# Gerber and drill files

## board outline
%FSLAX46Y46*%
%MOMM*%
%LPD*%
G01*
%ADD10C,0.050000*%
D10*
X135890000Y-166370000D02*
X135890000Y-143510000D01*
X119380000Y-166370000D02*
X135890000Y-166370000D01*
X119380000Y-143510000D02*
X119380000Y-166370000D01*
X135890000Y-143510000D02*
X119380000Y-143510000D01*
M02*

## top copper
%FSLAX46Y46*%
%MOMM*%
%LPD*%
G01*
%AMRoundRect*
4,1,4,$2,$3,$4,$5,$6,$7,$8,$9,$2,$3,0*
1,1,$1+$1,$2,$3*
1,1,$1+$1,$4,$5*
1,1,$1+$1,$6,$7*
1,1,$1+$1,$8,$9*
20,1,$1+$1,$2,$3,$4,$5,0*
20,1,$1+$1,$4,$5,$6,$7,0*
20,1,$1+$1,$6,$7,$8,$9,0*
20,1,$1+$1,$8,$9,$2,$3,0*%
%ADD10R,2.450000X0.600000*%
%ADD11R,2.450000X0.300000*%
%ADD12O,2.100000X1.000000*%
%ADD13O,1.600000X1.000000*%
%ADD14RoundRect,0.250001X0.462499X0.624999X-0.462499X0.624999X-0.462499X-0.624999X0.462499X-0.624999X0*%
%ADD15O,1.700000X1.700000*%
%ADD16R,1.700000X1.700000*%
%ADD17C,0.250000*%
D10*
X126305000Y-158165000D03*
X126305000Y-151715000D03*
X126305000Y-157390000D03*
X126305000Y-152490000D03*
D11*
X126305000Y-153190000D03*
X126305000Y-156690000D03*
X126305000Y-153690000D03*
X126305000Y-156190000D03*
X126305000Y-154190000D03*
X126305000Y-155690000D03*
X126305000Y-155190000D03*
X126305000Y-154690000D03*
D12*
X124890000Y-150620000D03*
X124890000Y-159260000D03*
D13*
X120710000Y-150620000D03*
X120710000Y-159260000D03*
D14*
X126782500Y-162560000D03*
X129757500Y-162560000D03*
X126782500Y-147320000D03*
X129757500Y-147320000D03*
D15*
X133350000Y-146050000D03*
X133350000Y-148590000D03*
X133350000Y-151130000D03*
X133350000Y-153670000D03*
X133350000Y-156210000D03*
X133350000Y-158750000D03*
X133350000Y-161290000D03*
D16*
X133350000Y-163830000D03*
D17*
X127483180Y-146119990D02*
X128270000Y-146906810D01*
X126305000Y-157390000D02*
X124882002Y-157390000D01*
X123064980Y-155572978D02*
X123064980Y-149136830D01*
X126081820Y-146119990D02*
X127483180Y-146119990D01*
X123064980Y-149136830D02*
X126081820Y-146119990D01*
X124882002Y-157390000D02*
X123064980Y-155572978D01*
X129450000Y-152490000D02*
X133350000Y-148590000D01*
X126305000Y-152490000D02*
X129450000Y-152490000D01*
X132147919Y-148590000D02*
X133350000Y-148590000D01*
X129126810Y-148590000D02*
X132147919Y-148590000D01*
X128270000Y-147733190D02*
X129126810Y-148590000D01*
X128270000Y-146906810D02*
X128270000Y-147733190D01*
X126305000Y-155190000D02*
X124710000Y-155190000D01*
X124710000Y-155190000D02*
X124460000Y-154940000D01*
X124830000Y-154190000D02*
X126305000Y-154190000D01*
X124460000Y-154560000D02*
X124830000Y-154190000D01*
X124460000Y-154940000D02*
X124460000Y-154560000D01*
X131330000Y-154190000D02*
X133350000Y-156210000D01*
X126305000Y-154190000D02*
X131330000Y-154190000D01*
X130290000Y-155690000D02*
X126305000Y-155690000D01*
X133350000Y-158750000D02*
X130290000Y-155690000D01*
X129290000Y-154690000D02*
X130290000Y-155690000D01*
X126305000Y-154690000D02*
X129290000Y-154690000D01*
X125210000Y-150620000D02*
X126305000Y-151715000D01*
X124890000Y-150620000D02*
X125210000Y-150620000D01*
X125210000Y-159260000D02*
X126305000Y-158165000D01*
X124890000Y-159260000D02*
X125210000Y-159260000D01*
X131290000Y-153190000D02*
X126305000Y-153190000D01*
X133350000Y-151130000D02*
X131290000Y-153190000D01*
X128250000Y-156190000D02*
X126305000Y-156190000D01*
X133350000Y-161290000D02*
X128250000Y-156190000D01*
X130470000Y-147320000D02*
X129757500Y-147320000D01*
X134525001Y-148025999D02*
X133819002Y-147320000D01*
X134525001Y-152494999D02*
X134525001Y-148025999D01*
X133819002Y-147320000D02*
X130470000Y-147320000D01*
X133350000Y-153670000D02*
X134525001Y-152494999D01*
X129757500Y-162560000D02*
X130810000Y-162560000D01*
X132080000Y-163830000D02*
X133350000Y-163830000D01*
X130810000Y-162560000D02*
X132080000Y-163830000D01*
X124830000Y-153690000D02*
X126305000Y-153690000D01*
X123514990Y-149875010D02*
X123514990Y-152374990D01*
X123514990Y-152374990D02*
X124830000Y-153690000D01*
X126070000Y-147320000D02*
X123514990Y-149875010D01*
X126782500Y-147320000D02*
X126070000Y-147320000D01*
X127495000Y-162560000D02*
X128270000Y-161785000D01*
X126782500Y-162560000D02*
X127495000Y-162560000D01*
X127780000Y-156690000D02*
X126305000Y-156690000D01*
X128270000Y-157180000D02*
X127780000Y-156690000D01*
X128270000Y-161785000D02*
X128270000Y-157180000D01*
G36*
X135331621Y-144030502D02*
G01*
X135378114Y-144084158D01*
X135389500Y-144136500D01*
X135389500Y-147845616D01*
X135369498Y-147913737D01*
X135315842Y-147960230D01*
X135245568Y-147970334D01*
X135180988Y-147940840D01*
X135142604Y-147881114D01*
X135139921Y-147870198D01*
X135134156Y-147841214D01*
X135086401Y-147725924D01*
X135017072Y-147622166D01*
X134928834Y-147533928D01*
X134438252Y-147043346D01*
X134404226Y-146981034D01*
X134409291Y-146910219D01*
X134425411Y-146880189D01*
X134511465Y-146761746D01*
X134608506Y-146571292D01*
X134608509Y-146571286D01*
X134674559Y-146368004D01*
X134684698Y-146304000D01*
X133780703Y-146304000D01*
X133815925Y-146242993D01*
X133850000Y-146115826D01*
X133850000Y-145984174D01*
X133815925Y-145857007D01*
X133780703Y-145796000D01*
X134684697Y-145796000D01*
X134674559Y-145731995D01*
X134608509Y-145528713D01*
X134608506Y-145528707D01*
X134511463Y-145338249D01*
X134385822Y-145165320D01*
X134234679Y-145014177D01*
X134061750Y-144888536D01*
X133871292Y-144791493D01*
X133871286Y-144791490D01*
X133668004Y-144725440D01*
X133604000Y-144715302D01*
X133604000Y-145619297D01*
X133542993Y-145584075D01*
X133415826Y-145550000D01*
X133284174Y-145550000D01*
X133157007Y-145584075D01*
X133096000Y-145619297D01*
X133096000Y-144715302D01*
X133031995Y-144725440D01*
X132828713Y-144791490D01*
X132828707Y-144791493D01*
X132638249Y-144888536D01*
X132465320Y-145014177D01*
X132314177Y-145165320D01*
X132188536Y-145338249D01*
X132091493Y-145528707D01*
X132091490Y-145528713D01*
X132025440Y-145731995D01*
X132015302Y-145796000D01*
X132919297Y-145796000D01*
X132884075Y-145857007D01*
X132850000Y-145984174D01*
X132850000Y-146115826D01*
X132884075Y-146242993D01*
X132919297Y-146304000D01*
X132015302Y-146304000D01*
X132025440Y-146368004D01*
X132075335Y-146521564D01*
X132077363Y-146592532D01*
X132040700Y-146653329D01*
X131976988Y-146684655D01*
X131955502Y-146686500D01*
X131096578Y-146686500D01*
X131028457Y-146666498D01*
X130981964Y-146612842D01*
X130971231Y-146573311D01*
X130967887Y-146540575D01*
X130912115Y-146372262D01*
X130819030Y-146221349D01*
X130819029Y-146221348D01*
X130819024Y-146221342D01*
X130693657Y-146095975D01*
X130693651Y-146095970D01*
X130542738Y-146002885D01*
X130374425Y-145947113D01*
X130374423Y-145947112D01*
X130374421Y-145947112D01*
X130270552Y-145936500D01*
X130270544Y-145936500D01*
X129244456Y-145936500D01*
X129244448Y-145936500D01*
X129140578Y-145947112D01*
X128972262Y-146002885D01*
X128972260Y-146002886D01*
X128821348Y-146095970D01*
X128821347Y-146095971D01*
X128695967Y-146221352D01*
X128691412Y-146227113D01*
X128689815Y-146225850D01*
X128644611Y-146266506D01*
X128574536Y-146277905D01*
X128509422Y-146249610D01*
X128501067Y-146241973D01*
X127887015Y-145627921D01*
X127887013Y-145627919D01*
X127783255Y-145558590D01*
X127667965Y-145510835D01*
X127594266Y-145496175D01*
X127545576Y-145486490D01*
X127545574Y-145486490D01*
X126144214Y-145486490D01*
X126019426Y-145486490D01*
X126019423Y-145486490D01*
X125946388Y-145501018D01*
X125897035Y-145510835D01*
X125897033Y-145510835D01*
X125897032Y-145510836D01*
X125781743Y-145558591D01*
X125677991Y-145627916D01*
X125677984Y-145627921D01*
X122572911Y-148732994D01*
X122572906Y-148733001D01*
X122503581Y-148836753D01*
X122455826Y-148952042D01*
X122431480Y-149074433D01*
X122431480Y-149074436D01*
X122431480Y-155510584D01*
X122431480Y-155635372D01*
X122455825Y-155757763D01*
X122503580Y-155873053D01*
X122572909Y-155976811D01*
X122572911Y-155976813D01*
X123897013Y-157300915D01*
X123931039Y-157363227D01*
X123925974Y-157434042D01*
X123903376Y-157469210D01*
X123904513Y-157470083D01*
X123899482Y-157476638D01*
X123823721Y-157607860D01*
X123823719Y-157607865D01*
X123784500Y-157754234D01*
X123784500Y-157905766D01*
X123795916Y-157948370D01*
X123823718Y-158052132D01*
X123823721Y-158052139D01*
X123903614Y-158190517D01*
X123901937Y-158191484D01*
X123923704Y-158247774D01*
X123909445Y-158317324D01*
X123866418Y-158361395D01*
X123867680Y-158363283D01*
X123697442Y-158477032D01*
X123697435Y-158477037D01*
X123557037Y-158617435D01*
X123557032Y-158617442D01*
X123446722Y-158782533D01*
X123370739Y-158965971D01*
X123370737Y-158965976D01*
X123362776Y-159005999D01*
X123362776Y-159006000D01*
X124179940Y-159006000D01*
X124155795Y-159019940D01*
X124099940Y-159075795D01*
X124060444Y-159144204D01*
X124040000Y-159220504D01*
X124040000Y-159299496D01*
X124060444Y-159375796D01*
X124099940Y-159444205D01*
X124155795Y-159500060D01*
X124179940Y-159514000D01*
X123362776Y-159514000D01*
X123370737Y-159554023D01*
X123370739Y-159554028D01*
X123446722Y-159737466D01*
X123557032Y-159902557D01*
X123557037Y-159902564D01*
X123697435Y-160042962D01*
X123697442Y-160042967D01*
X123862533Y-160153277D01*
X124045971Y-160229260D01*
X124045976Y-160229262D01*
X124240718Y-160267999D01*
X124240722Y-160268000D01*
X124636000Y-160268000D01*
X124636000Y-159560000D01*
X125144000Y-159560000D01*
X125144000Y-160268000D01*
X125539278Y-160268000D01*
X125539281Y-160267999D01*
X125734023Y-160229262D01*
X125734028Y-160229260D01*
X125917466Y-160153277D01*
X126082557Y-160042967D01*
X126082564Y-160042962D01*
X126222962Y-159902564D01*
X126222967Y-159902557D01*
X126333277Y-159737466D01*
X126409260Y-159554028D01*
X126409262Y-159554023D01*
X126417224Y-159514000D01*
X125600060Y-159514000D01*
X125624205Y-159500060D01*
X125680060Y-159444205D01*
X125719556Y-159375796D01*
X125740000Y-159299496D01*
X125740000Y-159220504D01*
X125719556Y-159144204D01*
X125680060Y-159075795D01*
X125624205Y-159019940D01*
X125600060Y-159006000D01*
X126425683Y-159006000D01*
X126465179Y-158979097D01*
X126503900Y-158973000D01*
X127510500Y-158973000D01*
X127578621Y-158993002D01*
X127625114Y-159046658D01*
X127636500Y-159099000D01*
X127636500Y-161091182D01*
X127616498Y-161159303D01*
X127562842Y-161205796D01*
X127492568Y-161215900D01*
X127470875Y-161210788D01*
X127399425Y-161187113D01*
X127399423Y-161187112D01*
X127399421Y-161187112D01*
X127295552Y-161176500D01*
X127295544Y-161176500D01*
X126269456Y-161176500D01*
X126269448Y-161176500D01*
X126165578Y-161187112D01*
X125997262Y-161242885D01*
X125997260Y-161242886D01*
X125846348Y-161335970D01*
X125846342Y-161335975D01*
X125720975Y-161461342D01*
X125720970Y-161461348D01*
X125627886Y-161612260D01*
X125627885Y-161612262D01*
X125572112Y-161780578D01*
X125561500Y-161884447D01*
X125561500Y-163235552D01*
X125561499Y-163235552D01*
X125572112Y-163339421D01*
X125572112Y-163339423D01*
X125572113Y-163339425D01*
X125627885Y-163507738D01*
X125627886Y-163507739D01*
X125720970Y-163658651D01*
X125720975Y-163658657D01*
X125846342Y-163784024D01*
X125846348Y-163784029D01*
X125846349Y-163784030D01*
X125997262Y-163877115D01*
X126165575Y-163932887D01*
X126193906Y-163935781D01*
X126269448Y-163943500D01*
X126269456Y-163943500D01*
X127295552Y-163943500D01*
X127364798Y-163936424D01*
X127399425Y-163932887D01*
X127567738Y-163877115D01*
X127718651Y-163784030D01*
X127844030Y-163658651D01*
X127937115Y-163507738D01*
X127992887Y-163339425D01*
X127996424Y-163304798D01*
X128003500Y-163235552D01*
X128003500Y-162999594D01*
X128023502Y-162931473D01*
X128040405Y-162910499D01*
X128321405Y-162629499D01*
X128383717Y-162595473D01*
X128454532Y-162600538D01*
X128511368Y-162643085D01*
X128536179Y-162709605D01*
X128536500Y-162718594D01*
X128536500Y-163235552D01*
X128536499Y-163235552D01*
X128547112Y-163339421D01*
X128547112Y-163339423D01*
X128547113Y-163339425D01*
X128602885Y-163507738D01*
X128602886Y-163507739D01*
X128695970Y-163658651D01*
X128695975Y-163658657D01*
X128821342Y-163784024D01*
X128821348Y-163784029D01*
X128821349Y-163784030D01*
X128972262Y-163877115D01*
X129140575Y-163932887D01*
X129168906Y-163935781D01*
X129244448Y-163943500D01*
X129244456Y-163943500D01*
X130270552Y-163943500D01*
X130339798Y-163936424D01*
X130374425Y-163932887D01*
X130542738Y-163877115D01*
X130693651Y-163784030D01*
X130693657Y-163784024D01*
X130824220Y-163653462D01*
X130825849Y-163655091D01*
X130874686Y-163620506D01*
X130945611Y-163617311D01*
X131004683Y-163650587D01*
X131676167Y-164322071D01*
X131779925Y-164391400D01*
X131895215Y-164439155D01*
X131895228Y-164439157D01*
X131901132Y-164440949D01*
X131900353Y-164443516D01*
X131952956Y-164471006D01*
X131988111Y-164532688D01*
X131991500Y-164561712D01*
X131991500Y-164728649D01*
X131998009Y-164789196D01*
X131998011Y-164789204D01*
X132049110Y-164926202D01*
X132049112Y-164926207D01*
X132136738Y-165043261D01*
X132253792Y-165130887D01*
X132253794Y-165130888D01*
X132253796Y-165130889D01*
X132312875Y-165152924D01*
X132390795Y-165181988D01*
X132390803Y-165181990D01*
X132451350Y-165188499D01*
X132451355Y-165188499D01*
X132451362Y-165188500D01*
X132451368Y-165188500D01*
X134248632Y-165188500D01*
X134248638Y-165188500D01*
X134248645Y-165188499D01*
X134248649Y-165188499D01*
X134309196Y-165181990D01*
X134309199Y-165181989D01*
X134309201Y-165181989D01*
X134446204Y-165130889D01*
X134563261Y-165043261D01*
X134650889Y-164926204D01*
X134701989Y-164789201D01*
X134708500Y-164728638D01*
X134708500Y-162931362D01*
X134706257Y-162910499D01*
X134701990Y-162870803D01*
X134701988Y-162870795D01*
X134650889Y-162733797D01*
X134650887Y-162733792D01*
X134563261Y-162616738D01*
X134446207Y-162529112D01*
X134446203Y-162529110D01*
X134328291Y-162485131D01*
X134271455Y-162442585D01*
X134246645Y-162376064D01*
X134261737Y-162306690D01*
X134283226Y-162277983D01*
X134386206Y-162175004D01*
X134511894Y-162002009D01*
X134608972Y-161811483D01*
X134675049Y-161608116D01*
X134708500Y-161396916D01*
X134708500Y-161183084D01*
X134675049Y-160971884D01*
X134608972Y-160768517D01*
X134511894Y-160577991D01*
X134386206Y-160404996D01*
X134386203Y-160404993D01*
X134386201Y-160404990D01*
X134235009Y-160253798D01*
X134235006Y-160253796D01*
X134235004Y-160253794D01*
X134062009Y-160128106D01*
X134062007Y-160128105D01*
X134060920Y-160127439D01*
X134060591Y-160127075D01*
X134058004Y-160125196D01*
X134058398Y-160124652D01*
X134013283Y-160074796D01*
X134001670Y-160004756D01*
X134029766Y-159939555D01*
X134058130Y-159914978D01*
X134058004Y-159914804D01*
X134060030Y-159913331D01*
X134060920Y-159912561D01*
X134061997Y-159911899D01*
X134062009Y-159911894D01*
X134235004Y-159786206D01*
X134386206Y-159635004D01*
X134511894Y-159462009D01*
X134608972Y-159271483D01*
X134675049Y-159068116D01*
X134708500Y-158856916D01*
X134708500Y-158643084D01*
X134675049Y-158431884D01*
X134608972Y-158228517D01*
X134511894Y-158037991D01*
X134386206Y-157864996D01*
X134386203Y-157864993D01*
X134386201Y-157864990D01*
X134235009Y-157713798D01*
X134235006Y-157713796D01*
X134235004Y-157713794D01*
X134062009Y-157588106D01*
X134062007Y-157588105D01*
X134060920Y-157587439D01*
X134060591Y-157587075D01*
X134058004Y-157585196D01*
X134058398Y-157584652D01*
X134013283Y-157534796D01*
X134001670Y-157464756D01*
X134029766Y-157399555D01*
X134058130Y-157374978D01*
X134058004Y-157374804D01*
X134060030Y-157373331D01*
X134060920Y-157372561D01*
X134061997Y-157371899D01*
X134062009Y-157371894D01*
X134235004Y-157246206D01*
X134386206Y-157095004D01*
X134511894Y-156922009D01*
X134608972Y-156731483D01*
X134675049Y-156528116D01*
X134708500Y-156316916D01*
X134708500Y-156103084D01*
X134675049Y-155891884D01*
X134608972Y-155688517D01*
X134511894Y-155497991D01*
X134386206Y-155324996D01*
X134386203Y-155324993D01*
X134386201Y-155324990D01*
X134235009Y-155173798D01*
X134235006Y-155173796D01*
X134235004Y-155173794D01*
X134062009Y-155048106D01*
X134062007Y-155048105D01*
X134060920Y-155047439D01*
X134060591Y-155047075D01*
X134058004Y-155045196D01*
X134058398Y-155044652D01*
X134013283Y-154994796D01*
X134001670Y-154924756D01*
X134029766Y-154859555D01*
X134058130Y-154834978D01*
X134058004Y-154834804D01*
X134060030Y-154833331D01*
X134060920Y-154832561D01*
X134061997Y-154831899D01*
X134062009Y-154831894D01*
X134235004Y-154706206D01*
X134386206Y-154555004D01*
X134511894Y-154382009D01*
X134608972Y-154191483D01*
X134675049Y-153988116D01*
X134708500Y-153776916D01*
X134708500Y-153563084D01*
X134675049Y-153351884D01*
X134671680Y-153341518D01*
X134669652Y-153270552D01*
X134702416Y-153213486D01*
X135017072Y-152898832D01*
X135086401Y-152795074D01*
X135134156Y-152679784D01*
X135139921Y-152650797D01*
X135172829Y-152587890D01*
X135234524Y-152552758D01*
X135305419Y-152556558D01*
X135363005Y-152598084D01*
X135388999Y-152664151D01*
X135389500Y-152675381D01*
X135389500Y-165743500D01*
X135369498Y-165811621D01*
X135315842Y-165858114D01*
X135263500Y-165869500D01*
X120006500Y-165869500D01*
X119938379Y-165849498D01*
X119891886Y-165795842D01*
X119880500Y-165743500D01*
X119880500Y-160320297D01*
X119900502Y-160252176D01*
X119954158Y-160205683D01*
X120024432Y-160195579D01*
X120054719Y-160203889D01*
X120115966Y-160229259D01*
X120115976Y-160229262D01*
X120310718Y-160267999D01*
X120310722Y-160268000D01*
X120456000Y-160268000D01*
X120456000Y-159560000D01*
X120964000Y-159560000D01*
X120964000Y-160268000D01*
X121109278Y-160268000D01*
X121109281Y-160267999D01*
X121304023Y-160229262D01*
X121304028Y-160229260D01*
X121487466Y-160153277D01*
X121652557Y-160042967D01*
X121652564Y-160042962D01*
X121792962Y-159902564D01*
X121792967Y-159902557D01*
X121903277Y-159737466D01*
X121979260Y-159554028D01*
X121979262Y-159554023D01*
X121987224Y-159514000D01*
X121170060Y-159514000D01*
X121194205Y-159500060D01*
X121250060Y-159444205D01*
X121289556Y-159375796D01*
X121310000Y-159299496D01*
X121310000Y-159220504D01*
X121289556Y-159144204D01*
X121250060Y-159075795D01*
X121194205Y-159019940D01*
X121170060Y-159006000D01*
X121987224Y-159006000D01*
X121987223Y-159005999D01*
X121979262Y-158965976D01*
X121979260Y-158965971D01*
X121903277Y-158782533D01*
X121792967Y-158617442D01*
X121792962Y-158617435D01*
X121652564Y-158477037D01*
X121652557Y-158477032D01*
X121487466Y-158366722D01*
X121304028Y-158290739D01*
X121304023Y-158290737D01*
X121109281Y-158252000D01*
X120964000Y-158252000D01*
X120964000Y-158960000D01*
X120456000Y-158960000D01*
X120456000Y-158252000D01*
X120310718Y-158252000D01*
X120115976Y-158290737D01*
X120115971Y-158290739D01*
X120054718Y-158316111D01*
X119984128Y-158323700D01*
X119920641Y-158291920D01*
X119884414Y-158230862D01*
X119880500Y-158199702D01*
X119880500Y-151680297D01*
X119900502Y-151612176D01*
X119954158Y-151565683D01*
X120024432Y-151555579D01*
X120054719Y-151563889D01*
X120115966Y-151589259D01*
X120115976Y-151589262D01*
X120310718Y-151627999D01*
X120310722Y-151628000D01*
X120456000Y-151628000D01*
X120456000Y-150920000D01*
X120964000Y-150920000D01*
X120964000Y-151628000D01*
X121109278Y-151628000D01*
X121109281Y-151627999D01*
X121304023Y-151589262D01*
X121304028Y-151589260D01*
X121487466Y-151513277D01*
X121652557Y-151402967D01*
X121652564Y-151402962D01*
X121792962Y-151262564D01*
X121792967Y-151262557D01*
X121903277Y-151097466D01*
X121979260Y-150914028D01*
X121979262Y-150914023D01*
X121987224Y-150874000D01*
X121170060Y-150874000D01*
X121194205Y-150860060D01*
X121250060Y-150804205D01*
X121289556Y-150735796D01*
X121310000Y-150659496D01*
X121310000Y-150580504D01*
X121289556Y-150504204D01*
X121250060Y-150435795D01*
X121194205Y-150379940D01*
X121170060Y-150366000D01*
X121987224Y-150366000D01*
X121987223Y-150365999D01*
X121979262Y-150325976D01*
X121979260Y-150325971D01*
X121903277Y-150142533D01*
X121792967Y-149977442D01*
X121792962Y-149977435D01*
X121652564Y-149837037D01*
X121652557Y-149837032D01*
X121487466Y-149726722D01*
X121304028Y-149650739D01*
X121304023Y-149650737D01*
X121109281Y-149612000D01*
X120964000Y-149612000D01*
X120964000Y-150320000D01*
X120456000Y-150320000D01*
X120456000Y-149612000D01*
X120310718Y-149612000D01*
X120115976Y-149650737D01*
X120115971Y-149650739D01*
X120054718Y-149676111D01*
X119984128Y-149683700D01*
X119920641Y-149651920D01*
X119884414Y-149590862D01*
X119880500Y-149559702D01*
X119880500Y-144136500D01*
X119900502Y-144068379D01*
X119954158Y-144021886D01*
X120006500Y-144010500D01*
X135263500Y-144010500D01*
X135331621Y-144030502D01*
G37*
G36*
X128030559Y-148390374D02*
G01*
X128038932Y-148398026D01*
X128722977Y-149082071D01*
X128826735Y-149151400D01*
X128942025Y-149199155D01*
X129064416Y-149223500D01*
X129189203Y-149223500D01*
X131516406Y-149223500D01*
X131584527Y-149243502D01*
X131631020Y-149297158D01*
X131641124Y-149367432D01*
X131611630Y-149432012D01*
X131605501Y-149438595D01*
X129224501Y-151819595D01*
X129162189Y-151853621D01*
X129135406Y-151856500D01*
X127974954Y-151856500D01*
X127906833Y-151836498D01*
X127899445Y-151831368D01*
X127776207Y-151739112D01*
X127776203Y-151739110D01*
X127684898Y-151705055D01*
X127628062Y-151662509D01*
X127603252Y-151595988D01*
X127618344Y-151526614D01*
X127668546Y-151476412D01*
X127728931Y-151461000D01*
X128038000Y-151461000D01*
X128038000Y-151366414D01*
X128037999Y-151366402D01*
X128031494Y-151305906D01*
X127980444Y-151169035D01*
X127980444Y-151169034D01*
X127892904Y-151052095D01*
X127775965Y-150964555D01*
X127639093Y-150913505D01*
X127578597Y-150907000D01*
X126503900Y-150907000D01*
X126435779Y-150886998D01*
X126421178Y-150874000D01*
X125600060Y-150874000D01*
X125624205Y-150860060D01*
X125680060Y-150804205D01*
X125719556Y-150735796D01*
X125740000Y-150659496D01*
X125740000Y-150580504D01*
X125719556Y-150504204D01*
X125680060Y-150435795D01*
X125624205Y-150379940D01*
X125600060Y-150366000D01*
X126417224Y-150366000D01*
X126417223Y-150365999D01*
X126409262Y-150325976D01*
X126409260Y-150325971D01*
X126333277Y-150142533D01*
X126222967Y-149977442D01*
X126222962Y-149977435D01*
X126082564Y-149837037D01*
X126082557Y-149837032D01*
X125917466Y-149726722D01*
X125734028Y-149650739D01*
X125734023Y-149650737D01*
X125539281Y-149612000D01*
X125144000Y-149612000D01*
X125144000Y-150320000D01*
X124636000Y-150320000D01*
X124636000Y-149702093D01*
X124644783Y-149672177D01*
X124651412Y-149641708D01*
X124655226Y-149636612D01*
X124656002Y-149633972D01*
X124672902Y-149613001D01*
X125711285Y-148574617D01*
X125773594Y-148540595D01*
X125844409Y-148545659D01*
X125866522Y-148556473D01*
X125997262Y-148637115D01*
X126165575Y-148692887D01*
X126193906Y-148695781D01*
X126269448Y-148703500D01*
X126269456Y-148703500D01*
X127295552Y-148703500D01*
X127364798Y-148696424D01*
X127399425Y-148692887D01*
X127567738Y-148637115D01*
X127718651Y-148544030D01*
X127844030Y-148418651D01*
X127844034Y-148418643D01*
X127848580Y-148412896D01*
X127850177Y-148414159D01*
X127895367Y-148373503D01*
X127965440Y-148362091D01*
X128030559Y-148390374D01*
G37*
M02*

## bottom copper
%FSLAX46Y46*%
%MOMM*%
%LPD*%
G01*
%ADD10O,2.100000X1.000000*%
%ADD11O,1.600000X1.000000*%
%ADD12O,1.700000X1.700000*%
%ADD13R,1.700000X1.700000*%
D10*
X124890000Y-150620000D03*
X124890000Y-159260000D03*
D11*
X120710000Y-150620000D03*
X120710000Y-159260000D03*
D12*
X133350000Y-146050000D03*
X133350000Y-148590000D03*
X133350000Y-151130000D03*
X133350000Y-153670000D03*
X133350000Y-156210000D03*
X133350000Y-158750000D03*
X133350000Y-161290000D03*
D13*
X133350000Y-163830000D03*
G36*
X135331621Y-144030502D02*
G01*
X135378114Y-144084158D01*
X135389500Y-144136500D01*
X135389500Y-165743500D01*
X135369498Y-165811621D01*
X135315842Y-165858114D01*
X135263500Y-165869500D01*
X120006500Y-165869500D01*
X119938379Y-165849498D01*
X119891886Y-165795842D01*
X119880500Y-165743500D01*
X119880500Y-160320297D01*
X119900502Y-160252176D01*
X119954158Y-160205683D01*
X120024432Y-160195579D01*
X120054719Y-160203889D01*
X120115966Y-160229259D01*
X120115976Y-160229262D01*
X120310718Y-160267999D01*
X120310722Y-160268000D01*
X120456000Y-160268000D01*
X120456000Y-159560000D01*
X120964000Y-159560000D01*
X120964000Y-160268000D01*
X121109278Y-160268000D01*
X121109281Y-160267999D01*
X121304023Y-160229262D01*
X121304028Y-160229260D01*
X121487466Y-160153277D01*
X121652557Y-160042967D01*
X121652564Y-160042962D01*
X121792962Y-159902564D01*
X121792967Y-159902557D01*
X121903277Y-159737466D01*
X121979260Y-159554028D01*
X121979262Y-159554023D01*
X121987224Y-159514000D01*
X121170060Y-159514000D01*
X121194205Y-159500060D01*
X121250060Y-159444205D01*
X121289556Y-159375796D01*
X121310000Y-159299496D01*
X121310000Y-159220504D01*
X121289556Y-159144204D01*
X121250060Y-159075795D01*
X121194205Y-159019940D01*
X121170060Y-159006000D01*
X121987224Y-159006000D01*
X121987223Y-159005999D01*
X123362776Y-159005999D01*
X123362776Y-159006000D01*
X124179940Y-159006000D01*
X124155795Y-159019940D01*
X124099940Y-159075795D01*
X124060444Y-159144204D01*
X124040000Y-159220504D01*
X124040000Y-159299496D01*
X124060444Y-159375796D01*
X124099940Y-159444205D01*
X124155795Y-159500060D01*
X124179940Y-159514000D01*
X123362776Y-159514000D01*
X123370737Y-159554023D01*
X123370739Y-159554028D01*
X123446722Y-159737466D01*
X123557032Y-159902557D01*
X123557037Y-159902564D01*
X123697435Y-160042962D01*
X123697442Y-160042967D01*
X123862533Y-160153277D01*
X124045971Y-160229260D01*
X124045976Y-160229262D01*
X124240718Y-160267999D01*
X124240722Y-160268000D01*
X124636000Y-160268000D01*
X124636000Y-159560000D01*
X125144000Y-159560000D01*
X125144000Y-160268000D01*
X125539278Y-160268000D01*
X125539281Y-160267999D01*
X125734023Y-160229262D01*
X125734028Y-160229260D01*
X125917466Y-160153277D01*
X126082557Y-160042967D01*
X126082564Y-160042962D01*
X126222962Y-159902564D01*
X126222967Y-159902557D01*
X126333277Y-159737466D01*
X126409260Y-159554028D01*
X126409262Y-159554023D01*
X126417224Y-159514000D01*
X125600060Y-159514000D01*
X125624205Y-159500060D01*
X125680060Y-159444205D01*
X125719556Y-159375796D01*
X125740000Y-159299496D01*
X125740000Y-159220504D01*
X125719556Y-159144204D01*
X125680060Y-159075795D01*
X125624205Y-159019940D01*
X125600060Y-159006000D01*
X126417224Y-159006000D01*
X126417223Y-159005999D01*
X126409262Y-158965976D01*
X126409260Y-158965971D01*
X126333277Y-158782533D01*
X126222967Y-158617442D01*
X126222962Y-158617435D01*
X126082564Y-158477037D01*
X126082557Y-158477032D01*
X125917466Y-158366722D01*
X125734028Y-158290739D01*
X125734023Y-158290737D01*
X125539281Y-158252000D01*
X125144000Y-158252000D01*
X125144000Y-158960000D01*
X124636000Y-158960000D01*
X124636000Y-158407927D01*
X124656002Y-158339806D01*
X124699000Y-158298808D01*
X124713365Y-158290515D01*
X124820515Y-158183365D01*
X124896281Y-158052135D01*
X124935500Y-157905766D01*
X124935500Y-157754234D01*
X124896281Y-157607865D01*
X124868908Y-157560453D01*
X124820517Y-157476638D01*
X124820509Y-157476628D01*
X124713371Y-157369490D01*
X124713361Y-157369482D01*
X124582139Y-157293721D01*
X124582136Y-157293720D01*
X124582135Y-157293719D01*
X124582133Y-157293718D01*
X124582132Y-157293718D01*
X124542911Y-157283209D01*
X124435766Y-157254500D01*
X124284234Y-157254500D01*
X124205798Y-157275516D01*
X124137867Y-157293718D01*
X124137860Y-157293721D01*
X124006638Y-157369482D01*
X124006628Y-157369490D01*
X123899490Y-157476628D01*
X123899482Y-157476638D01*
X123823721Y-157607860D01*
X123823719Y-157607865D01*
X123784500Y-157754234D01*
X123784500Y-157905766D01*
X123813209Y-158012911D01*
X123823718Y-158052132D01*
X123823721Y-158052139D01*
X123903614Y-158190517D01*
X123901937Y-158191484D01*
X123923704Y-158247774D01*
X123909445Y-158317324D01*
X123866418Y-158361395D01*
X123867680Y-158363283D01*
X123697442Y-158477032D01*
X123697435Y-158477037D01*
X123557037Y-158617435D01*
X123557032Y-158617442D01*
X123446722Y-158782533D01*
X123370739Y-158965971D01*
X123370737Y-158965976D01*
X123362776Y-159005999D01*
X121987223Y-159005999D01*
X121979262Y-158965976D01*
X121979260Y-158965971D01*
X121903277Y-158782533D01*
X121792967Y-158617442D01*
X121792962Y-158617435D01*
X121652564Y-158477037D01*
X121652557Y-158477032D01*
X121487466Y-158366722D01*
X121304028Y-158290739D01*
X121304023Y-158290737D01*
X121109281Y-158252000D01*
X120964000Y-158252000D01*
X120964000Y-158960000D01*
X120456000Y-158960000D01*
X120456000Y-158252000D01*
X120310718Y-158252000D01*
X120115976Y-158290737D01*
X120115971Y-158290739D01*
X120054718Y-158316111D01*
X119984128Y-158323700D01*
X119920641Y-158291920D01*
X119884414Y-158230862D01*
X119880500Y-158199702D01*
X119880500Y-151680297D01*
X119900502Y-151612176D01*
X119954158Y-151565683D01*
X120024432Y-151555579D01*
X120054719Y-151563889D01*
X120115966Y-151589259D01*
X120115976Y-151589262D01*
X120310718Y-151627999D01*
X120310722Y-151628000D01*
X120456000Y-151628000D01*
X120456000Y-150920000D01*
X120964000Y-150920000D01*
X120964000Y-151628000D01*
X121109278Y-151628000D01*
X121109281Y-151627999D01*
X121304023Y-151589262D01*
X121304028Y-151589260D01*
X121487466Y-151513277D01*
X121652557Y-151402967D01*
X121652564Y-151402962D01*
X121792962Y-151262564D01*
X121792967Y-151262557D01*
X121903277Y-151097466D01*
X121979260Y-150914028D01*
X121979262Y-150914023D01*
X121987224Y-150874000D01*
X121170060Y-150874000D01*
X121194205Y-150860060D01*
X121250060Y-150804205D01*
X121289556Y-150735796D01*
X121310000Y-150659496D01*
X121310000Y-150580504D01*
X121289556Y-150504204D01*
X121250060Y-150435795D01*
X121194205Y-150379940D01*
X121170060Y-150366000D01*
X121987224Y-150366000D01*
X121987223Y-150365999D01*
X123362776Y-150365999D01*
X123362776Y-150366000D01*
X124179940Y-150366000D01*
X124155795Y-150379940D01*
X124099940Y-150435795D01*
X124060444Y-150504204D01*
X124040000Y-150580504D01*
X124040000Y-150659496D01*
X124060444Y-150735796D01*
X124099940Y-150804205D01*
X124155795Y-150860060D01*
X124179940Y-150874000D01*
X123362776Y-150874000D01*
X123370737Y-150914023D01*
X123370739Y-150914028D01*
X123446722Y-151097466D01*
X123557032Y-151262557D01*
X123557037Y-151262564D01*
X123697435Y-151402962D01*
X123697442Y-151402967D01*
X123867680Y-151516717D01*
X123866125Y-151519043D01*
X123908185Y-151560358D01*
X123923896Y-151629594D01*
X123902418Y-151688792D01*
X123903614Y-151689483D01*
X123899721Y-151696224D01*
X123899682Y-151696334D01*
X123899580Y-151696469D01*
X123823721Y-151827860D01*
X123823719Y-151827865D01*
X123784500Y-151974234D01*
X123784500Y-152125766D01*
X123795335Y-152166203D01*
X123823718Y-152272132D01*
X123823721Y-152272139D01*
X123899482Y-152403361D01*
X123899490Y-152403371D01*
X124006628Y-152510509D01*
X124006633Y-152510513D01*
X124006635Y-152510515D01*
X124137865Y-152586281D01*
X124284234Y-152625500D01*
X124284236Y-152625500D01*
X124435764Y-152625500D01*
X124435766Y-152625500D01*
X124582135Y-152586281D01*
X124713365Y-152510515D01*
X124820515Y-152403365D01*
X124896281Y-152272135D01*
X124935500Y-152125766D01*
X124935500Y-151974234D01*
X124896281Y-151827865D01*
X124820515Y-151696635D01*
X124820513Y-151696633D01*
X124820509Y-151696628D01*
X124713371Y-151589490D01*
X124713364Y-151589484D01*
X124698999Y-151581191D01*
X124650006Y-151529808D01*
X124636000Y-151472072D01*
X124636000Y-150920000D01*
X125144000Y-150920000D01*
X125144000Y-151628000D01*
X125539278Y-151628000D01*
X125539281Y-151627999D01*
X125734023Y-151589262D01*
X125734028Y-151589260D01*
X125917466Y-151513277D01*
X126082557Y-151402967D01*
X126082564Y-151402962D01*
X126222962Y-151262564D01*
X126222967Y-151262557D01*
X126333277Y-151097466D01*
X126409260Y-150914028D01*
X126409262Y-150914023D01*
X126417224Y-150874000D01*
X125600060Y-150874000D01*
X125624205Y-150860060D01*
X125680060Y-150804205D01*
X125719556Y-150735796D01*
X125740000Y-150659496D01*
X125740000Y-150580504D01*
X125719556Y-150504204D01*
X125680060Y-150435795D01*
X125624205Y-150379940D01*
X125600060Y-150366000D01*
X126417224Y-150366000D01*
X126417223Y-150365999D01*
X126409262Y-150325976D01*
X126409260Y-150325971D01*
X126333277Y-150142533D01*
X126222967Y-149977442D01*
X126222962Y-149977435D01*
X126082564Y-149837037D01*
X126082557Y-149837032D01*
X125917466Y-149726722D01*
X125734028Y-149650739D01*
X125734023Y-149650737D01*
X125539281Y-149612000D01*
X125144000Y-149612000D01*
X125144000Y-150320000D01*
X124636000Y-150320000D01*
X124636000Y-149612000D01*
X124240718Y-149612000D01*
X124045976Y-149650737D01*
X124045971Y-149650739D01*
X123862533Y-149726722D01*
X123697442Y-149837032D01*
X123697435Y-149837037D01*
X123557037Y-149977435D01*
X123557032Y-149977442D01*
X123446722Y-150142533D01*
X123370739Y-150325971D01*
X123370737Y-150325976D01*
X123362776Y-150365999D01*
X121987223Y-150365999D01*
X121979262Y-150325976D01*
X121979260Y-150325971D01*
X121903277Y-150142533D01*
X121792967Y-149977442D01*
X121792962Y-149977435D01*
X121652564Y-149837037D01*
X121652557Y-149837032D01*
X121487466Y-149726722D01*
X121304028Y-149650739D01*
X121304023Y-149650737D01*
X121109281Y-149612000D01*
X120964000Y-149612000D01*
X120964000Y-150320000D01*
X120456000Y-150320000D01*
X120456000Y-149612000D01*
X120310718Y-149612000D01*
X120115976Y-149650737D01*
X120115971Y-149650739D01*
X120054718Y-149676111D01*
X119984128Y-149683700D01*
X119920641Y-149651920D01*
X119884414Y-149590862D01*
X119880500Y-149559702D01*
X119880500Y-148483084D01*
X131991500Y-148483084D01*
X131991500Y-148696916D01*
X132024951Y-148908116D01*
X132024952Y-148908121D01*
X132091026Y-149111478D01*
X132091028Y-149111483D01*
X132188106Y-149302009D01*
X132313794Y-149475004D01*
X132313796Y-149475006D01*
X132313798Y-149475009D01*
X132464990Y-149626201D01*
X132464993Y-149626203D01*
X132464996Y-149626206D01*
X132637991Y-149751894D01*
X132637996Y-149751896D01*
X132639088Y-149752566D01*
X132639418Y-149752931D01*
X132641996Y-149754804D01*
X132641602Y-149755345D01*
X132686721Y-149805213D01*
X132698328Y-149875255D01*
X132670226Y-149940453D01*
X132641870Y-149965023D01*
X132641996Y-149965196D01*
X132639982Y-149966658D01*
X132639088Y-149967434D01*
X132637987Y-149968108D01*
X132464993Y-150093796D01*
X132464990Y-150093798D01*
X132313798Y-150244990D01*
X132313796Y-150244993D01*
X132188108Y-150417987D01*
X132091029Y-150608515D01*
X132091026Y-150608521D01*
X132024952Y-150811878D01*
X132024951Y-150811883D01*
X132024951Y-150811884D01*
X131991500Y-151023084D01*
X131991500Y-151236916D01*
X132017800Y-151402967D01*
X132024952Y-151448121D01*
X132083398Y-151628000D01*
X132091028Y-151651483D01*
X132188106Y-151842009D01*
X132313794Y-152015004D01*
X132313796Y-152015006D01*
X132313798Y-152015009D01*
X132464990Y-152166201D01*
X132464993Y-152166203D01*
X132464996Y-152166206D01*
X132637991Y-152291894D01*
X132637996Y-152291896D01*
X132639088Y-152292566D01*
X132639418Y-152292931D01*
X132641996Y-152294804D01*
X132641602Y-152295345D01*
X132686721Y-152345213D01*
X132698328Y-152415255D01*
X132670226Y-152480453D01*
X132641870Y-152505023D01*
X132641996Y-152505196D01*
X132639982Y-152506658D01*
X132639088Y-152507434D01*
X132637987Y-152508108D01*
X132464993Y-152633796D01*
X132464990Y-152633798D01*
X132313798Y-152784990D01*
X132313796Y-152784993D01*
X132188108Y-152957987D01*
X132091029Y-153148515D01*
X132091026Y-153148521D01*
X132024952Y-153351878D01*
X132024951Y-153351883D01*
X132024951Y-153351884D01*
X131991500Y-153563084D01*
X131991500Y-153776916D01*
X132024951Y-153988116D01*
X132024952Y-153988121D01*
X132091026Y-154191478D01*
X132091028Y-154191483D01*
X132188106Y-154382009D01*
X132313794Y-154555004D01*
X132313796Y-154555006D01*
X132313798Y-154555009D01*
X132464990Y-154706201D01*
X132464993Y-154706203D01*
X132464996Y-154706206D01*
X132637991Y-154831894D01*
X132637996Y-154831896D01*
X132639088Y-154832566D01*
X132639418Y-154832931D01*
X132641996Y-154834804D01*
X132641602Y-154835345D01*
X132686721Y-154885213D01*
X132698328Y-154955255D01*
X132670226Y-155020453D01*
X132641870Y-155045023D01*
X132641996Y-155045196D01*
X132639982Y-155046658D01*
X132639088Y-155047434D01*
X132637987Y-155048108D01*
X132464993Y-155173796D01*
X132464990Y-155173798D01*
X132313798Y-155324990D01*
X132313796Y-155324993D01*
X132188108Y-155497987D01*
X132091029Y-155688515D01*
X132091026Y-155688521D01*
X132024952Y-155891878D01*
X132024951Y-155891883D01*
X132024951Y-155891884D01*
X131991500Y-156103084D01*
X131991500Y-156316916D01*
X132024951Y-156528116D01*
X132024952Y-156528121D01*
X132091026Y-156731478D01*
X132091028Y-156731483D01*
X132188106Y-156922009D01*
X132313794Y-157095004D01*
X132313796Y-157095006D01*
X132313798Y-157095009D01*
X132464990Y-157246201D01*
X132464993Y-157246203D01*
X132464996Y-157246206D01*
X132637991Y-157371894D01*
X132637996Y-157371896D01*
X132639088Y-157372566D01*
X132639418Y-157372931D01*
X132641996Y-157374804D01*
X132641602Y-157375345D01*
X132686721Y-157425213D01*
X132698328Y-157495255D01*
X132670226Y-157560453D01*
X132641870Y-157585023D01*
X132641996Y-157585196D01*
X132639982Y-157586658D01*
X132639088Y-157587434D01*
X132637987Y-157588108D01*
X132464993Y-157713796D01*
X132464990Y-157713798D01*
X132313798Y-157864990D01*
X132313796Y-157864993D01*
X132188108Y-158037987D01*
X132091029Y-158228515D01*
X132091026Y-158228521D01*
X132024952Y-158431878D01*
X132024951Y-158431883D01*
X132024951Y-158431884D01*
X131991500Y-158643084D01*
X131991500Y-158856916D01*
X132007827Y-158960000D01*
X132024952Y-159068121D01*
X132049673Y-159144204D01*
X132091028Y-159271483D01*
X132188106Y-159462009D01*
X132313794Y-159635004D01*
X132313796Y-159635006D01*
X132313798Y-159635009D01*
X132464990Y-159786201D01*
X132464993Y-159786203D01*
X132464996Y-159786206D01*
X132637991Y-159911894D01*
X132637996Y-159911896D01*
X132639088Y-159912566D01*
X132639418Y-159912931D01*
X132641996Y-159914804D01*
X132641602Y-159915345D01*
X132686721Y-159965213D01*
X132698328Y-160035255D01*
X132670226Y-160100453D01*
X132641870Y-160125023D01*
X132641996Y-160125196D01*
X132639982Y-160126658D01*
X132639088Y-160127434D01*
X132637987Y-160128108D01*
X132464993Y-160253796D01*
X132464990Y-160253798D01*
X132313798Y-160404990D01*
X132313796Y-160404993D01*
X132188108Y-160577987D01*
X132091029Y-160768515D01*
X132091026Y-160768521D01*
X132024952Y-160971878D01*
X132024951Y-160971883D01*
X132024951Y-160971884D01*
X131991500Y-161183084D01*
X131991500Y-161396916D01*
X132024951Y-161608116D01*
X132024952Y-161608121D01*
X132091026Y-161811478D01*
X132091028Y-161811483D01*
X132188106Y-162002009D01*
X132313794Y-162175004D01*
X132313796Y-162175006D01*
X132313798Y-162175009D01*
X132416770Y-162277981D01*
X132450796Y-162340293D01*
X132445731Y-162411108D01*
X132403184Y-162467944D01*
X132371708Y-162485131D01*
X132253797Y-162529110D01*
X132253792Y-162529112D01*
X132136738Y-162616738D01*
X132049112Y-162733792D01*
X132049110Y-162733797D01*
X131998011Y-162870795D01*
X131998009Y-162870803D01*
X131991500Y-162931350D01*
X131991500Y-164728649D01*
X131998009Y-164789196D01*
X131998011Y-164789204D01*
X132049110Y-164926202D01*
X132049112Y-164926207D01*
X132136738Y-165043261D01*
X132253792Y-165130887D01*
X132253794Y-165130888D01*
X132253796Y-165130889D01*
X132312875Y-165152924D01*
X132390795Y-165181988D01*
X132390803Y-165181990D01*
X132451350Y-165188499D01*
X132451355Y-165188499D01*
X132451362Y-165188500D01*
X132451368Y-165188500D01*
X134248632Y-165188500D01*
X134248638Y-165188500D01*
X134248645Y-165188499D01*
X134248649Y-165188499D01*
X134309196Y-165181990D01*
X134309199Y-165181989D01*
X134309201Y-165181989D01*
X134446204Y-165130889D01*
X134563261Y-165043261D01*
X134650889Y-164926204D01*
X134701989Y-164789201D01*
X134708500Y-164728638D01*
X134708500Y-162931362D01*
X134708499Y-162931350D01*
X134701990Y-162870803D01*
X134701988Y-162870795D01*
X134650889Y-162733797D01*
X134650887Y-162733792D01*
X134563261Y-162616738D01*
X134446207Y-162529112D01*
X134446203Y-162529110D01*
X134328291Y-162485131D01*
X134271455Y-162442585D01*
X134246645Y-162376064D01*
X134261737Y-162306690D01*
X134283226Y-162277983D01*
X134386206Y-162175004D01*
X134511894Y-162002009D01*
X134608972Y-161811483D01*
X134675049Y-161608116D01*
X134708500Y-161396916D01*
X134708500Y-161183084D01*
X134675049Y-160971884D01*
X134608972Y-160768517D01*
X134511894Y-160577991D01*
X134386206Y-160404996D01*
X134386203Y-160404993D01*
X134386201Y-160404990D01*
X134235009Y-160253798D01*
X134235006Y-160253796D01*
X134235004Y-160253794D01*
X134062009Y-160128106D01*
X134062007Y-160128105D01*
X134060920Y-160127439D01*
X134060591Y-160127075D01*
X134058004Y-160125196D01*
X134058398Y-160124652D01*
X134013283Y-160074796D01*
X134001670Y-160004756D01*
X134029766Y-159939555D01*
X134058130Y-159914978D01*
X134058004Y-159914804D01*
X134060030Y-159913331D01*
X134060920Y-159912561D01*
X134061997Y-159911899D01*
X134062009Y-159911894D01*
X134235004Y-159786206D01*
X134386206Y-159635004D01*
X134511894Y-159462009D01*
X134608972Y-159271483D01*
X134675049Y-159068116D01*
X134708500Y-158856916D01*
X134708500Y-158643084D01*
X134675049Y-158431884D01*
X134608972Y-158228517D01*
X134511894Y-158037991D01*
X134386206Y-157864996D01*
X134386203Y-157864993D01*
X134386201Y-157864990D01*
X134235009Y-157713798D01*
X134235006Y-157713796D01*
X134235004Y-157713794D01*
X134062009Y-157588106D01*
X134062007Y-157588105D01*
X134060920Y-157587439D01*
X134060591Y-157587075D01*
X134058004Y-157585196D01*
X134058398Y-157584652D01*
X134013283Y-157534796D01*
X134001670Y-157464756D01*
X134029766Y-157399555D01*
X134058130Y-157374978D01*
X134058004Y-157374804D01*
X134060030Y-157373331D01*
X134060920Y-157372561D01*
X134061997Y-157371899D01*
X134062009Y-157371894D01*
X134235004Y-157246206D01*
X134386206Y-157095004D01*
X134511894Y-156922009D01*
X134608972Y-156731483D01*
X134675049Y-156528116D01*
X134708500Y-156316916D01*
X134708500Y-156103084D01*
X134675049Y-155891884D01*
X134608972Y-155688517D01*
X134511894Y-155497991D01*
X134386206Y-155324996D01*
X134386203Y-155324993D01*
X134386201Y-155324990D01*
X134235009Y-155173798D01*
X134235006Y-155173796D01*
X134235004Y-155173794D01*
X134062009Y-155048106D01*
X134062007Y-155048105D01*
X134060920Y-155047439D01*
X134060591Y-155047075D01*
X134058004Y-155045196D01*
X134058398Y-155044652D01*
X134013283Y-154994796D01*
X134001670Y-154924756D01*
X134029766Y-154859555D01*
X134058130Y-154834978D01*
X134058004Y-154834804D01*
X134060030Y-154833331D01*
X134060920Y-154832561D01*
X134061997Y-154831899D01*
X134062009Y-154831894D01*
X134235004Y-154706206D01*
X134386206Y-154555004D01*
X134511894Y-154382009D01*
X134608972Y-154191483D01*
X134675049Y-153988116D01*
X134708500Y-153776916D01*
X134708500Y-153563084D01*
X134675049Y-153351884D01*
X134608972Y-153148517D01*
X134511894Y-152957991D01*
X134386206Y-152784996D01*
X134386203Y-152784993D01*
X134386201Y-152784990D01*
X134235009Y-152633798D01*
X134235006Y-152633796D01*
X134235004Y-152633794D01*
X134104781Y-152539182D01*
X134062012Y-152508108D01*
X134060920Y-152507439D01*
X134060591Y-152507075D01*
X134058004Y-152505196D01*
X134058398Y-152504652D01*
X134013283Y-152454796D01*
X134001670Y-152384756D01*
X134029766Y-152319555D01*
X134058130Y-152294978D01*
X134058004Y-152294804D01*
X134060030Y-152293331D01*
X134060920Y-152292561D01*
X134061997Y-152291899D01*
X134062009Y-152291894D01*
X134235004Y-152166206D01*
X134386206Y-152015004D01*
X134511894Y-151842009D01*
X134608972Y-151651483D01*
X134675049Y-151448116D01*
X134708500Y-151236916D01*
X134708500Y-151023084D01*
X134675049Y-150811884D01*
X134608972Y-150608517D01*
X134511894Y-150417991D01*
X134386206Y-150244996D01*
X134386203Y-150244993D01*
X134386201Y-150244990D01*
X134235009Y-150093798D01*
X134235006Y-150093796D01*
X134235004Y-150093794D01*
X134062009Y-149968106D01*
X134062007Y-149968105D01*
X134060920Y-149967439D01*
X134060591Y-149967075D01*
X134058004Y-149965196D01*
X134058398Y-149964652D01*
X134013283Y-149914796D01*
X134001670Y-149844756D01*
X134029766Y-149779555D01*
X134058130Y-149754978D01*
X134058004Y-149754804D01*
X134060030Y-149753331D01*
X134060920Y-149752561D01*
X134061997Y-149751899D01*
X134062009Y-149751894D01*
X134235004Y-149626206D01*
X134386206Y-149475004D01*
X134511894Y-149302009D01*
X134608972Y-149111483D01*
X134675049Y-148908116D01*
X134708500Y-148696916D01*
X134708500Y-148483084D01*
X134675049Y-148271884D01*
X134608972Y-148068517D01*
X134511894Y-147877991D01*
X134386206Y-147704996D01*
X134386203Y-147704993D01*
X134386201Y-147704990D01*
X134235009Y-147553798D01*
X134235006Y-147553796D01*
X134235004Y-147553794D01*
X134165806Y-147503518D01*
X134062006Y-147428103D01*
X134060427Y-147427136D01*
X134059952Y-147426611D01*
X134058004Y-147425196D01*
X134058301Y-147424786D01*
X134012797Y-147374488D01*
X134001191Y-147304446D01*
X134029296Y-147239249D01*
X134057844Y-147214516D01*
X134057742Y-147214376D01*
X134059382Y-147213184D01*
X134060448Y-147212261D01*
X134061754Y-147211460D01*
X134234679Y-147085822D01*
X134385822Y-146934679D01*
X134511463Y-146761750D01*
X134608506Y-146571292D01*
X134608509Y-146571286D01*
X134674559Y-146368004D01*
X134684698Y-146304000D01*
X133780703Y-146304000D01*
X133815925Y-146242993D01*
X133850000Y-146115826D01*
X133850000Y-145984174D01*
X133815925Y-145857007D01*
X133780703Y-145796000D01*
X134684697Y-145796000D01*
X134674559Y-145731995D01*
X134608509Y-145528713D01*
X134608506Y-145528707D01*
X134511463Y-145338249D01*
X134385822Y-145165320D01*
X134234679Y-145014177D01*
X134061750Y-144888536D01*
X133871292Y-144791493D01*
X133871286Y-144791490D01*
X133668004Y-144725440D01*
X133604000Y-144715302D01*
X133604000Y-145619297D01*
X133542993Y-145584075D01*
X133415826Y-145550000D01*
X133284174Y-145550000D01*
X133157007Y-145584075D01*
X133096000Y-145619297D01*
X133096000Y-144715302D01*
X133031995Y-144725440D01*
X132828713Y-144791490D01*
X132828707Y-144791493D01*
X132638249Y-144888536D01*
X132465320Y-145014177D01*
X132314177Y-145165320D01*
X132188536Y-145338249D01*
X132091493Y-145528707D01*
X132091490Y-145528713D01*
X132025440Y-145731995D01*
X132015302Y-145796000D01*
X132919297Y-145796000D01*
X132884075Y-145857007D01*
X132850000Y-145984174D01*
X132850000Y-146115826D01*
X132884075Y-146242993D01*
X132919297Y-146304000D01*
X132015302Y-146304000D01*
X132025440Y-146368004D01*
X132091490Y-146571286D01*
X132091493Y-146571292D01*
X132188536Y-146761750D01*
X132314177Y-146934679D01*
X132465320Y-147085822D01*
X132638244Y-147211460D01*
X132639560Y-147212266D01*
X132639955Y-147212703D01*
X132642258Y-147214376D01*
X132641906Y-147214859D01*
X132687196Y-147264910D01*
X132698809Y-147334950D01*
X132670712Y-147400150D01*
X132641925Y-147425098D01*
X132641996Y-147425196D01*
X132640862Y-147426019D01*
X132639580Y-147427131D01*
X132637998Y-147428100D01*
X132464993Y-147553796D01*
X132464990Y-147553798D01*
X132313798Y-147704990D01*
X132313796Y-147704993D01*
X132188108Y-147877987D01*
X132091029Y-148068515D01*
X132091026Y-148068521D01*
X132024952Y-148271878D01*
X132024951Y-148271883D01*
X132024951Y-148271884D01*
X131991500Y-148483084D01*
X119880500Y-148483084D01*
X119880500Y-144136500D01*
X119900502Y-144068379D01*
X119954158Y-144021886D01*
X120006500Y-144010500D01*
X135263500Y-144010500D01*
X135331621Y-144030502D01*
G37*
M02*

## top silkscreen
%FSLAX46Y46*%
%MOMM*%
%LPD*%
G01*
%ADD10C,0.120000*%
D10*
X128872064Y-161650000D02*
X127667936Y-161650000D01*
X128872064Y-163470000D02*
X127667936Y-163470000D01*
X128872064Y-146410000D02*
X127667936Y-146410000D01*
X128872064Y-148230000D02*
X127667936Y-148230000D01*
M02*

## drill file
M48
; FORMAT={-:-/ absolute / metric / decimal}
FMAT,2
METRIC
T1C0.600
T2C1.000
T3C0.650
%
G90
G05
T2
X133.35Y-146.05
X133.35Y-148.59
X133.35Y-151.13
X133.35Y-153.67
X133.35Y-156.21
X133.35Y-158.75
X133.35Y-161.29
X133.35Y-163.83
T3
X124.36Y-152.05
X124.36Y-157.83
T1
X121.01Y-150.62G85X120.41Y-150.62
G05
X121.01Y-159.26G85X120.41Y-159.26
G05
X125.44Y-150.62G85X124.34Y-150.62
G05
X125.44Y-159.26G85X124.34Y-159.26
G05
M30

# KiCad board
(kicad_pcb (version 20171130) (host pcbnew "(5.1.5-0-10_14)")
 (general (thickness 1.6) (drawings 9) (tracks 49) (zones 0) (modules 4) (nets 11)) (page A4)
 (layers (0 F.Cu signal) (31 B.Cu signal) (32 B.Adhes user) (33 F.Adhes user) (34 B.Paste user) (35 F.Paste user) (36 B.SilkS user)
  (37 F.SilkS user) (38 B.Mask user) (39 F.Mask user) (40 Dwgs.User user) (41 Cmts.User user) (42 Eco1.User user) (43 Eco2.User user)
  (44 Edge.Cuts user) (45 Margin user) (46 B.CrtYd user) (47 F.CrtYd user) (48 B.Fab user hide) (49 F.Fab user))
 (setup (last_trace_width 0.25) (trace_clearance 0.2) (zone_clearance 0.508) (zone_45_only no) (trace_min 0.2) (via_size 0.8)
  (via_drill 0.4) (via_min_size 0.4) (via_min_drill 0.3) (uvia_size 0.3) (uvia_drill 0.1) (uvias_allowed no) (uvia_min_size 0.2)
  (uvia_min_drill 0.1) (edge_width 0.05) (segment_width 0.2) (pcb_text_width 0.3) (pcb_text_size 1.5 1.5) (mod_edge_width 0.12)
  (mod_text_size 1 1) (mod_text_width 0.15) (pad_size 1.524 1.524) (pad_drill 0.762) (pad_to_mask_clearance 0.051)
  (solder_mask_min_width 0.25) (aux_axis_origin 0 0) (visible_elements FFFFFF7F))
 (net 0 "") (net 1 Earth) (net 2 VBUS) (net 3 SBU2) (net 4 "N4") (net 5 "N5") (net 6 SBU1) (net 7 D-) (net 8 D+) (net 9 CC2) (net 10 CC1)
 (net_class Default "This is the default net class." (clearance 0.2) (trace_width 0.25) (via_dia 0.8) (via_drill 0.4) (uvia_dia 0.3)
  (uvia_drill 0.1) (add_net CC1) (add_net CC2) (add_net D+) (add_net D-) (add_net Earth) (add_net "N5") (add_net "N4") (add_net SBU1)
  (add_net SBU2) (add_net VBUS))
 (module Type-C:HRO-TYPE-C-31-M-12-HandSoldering (layer F.Cu) (at 118.11 154.94 270)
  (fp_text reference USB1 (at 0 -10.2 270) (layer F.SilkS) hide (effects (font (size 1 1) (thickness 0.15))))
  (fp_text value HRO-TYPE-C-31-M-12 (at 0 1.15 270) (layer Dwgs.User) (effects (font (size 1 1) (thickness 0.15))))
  (pad 12 smd rect (at 3.225 -8.195 270) (size 0.6 2.45) (layers F.Cu F.Paste F.Mask) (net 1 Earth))
  (pad 1 smd rect (at -3.225 -8.195 270) (size 0.6 2.45) (layers F.Cu F.Paste F.Mask) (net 1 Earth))
  (pad 11 smd rect (at 2.45 -8.195 270) (size 0.6 2.45) (layers F.Cu F.Paste F.Mask) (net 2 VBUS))
  (pad 2 smd rect (at -2.45 -8.195 270) (size 0.6 2.45) (layers F.Cu F.Paste F.Mask) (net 2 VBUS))
  (pad 3 smd rect (at -1.75 -8.195 270) (size 0.3 2.45) (layers F.Cu F.Paste F.Mask) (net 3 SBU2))
  (pad 10 smd rect (at 1.75 -8.195 270) (size 0.3 2.45) (layers F.Cu F.Paste F.Mask) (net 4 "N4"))
  (pad 4 smd rect (at -1.25 -8.195 270) (size 0.3 2.45) (layers F.Cu F.Paste F.Mask) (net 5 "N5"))
  (pad 9 smd rect (at 1.25 -8.195 270) (size 0.3 2.45) (layers F.Cu F.Paste F.Mask) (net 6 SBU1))
  (pad 5 smd rect (at -0.75 -8.195 270) (size 0.3 2.45) (layers F.Cu F.Paste F.Mask) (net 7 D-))
  (pad 8 smd rect (at 0.75 -8.195 270) (size 0.3 2.45) (layers F.Cu F.Paste F.Mask) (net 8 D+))
  (pad 7 smd rect (at 0.25 -8.195 270) (size 0.3 2.45) (layers F.Cu F.Paste F.Mask) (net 7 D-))
  (pad 6 smd rect (at -0.25 -8.195 270) (size 0.3 2.45) (layers F.Cu F.Paste F.Mask) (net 8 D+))
  (pad "" np_thru_hole circle (at 2.89 -6.25 270) (size 0.65 0.65) (drill 0.65) (layers *.Cu *.Mask))
  (pad "" np_thru_hole circle (at -2.89 -6.25 270) (size 0.65 0.65) (drill 0.65) (layers *.Cu *.Mask))
  (pad 13 thru_hole oval (at -4.32 -6.78 270) (size 1 2.1) (drill oval 0.6 1.7) (layers *.Cu B.Mask) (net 1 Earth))
  (pad 13 thru_hole oval (at 4.32 -6.78 270) (size 1 2.1) (drill oval 0.6 1.7) (layers *.Cu B.Mask) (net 1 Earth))
  (pad 13 thru_hole oval (at -4.32 -2.6 270) (size 1 1.6) (drill oval 0.6 1.2) (layers *.Cu B.Mask) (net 1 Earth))
  (pad 13 thru_hole oval (at 4.32 -2.6 270) (size 1 1.6) (drill oval 0.6 1.2) (layers *.Cu B.Mask) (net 1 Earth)))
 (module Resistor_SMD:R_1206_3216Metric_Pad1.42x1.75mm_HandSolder (layer F.Cu) (at 128.27 162.56 180)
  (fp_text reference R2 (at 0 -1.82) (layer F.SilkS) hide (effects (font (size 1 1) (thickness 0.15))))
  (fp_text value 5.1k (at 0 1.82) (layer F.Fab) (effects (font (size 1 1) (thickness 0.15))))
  (fp_line (start -0.602064 0.91) (end 0.602064 0.91) (layer F.SilkS) (width 0.12))
  (fp_line (start -0.602064 -0.91) (end 0.602064 -0.91) (layer F.SilkS) (width 0.12))
  (pad 2 smd roundrect (at 1.4875 0 180) (size 1.425 1.75) (layers F.Cu F.Paste F.Mask) (roundrect_rratio 0.175439) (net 4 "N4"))
  (pad 1 smd roundrect (at -1.4875 0 180) (size 1.425 1.75) (layers F.Cu F.Paste F.Mask) (roundrect_rratio 0.175439) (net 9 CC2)))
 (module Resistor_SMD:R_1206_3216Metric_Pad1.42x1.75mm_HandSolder (layer F.Cu) (at 128.27 147.32 180)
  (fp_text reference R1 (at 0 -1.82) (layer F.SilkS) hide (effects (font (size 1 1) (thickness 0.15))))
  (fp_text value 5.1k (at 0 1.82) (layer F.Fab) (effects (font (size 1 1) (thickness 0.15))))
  (fp_line (start -0.602064 0.91) (end 0.602064 0.91) (layer F.SilkS) (width 0.12))
  (fp_line (start -0.602064 -0.91) (end 0.602064 -0.91) (layer F.SilkS) (width 0.12))
  (pad 2 smd roundrect (at 1.4875 0 180) (size 1.425 1.75) (layers F.Cu F.Paste F.Mask) (roundrect_rratio 0.175439) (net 5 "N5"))
  (pad 1 smd roundrect (at -1.4875 0 180) (size 1.425 1.75) (layers F.Cu F.Paste F.Mask) (roundrect_rratio 0.175439) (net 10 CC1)))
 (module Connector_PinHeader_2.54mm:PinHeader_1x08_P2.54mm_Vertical (layer B.Cu) (at 133.35 163.83)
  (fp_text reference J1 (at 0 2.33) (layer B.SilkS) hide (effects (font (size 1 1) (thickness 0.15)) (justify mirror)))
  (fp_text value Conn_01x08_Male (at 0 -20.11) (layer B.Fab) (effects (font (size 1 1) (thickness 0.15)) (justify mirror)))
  (pad 8 thru_hole oval (at 0 -17.78) (size 1.7 1.7) (drill 1) (layers *.Cu *.Mask) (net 1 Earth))
  (pad 7 thru_hole oval (at 0 -15.24) (size 1.7 1.7) (drill 1) (layers *.Cu *.Mask) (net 2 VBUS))
  (pad 6 thru_hole oval (at 0 -12.7) (size 1.7 1.7) (drill 1) (layers *.Cu *.Mask) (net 3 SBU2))
  (pad 5 thru_hole oval (at 0 -10.16) (size 1.7 1.7) (drill 1) (layers *.Cu *.Mask) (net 10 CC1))
  (pad 4 thru_hole oval (at 0 -7.62) (size 1.7 1.7) (drill 1) (layers *.Cu *.Mask) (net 7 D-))
  (pad 3 thru_hole oval (at 0 -5.08) (size 1.7 1.7) (drill 1) (layers *.Cu *.Mask) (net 8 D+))
  (pad 2 thru_hole oval (at 0 -2.54) (size 1.7 1.7) (drill 1) (layers *.Cu *.Mask) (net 6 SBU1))
  (pad 1 thru_hole rect (at 0 0) (size 1.7 1.7) (drill 1) (layers *.Cu *.Mask) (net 9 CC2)))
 (gr_line (start 135.89 166.37) (end 135.89 143.51) (layer Edge.Cuts) (width 0.05))
 (gr_line (start 119.38 166.37) (end 135.89 166.37) (layer Edge.Cuts) (width 0.05))
 (gr_line (start 119.38 143.51) (end 119.38 166.37) (layer Edge.Cuts) (width 0.05))
 (gr_line (start 135.89 143.51) (end 119.38 143.51) (layer Edge.Cuts) (width 0.05))
 (segment (start 127.48318 146.11999) (end 128.27 146.90681) (width 0.25) (layer F.Cu) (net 2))
 (segment (start 126.305 157.39) (end 124.882002 157.39) (width 0.25) (layer F.Cu) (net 2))
 (segment (start 123.06498 155.572978) (end 123.06498 149.13683) (width 0.25) (layer F.Cu) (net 2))
 (segment (start 126.08182 146.11999) (end 127.48318 146.11999) (width 0.25) (layer F.Cu) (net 2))
 (segment (start 123.06498 149.13683) (end 126.08182 146.11999) (width 0.25) (layer F.Cu) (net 2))
 (segment (start 124.882002 157.39) (end 123.06498 155.572978) (width 0.25) (layer F.Cu) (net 2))
 (segment (start 129.45 152.49) (end 133.35 148.59) (width 0.25) (layer F.Cu) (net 2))
 (segment (start 126.305 152.49) (end 129.45 152.49) (width 0.25) (layer F.Cu) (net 2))
 (segment (start 132.147919 148.59) (end 133.35 148.59) (width 0.25) (layer F.Cu) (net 2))
 (segment (start 129.12681 148.59) (end 132.147919 148.59) (width 0.25) (layer F.Cu) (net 2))
 (segment (start 128.27 147.73319) (end 129.12681 148.59) (width 0.25) (layer F.Cu) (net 2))
 (segment (start 128.27 146.90681) (end 128.27 147.73319) (width 0.25) (layer F.Cu) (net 2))
 (segment (start 126.305 155.19) (end 124.71 155.19) (width 0.25) (layer F.Cu) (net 7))
 (segment (start 124.71 155.19) (end 124.46 154.94) (width 0.25) (layer F.Cu) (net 7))
 (segment (start 124.83 154.19) (end 126.305 154.19) (width 0.25) (layer F.Cu) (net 7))
 (segment (start 124.46 154.56) (end 124.83 154.19) (width 0.25) (layer F.Cu) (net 7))
 (segment (start 124.46 154.94) (end 124.46 154.56) (width 0.25) (layer F.Cu) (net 7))
 (segment (start 131.33 154.19) (end 133.35 156.21) (width 0.25) (layer F.Cu) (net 7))
 (segment (start 126.305 154.19) (end 131.33 154.19) (width 0.25) (layer F.Cu) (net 7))
 (segment (start 130.29 155.69) (end 126.305 155.69) (width 0.25) (layer F.Cu) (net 8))
 (segment (start 133.35 158.75) (end 130.29 155.69) (width 0.25) (layer F.Cu) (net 8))
 (segment (start 129.29 154.69) (end 130.29 155.69) (width 0.25) (layer F.Cu) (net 8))
 (segment (start 126.305 154.69) (end 129.29 154.69) (width 0.25) (layer F.Cu) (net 8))
 (segment (start 125.21 150.62) (end 126.305 151.715) (width 0.25) (layer F.Cu) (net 1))
 (segment (start 124.89 150.62) (end 125.21 150.62) (width 0.25) (layer F.Cu) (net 1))
 (segment (start 125.21 159.26) (end 126.305 158.165) (width 0.25) (layer F.Cu) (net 1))
 (segment (start 124.89 159.26) (end 125.21 159.26) (width 0.25) (layer F.Cu) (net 1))
 (segment (start 131.29 153.19) (end 126.305 153.19) (width 0.25) (layer F.Cu) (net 3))
 (segment (start 133.35 151.13) (end 131.29 153.19) (width 0.25) (layer F.Cu) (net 3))
 (segment (start 128.25 156.19) (end 126.305 156.19) (width 0.25) (layer F.Cu) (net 6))
 (segment (start 133.35 161.29) (end 128.25 156.19) (width 0.25) (layer F.Cu) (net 6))
 (segment (start 130.47 147.32) (end 129.7575 147.32) (width 0.25) (layer F.Cu) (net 10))
 (segment (start 134.525001 148.025999) (end 133.819002 147.32) (width 0.25) (layer F.Cu) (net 10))
 (segment (start 134.525001 152.494999) (end 134.525001 148.025999) (width 0.25) (layer F.Cu) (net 10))
 (segment (start 133.819002 147.32) (end 130.47 147.32) (width 0.25) (layer F.Cu) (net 10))
 (segment (start 133.35 153.67) (end 134.525001 152.494999) (width 0.25) (layer F.Cu) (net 10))
 (segment (start 129.7575 162.56) (end 130.81 162.56) (width 0.25) (layer F.Cu) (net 9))
 (segment (start 132.08 163.83) (end 133.35 163.83) (width 0.25) (layer F.Cu) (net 9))
 (segment (start 130.81 162.56) (end 132.08 163.83) (width 0.25) (layer F.Cu) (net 9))
 (segment (start 124.83 153.69) (end 126.305 153.69) (width 0.25) (layer F.Cu) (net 5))
 (segment (start 123.51499 149.87501) (end 123.51499 152.37499) (width 0.25) (layer F.Cu) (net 5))
 (segment (start 123.51499 152.37499) (end 124.83 153.69) (width 0.25) (layer F.Cu) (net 5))
 (segment (start 126.07 147.32) (end 123.51499 149.87501) (width 0.25) (layer F.Cu) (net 5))
 (segment (start 126.7825 147.32) (end 126.07 147.32) (width 0.25) (layer F.Cu) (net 5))
 (segment (start 127.495 162.56) (end 128.27 161.785) (width 0.25) (layer F.Cu) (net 4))
 (segment (start 126.7825 162.56) (end 127.495 162.56) (width 0.25) (layer F.Cu) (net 4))
 (segment (start 127.78 156.69) (end 126.305 156.69) (width 0.25) (layer F.Cu) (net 4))
 (segment (start 128.27 157.18) (end 127.78 156.69) (width 0.25) (layer F.Cu) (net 4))
 (segment (start 128.27 161.785) (end 128.27 157.18) (width 0.25) (layer F.Cu) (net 4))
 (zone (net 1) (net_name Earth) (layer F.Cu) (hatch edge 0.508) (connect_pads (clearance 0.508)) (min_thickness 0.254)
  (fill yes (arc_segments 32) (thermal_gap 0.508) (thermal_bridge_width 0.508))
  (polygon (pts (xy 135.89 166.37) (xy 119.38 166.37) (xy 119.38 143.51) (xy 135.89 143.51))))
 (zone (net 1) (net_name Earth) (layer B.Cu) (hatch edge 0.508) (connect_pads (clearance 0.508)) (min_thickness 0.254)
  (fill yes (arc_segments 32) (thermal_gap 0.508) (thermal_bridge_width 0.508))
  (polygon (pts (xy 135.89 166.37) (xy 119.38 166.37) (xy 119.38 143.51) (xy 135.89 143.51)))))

